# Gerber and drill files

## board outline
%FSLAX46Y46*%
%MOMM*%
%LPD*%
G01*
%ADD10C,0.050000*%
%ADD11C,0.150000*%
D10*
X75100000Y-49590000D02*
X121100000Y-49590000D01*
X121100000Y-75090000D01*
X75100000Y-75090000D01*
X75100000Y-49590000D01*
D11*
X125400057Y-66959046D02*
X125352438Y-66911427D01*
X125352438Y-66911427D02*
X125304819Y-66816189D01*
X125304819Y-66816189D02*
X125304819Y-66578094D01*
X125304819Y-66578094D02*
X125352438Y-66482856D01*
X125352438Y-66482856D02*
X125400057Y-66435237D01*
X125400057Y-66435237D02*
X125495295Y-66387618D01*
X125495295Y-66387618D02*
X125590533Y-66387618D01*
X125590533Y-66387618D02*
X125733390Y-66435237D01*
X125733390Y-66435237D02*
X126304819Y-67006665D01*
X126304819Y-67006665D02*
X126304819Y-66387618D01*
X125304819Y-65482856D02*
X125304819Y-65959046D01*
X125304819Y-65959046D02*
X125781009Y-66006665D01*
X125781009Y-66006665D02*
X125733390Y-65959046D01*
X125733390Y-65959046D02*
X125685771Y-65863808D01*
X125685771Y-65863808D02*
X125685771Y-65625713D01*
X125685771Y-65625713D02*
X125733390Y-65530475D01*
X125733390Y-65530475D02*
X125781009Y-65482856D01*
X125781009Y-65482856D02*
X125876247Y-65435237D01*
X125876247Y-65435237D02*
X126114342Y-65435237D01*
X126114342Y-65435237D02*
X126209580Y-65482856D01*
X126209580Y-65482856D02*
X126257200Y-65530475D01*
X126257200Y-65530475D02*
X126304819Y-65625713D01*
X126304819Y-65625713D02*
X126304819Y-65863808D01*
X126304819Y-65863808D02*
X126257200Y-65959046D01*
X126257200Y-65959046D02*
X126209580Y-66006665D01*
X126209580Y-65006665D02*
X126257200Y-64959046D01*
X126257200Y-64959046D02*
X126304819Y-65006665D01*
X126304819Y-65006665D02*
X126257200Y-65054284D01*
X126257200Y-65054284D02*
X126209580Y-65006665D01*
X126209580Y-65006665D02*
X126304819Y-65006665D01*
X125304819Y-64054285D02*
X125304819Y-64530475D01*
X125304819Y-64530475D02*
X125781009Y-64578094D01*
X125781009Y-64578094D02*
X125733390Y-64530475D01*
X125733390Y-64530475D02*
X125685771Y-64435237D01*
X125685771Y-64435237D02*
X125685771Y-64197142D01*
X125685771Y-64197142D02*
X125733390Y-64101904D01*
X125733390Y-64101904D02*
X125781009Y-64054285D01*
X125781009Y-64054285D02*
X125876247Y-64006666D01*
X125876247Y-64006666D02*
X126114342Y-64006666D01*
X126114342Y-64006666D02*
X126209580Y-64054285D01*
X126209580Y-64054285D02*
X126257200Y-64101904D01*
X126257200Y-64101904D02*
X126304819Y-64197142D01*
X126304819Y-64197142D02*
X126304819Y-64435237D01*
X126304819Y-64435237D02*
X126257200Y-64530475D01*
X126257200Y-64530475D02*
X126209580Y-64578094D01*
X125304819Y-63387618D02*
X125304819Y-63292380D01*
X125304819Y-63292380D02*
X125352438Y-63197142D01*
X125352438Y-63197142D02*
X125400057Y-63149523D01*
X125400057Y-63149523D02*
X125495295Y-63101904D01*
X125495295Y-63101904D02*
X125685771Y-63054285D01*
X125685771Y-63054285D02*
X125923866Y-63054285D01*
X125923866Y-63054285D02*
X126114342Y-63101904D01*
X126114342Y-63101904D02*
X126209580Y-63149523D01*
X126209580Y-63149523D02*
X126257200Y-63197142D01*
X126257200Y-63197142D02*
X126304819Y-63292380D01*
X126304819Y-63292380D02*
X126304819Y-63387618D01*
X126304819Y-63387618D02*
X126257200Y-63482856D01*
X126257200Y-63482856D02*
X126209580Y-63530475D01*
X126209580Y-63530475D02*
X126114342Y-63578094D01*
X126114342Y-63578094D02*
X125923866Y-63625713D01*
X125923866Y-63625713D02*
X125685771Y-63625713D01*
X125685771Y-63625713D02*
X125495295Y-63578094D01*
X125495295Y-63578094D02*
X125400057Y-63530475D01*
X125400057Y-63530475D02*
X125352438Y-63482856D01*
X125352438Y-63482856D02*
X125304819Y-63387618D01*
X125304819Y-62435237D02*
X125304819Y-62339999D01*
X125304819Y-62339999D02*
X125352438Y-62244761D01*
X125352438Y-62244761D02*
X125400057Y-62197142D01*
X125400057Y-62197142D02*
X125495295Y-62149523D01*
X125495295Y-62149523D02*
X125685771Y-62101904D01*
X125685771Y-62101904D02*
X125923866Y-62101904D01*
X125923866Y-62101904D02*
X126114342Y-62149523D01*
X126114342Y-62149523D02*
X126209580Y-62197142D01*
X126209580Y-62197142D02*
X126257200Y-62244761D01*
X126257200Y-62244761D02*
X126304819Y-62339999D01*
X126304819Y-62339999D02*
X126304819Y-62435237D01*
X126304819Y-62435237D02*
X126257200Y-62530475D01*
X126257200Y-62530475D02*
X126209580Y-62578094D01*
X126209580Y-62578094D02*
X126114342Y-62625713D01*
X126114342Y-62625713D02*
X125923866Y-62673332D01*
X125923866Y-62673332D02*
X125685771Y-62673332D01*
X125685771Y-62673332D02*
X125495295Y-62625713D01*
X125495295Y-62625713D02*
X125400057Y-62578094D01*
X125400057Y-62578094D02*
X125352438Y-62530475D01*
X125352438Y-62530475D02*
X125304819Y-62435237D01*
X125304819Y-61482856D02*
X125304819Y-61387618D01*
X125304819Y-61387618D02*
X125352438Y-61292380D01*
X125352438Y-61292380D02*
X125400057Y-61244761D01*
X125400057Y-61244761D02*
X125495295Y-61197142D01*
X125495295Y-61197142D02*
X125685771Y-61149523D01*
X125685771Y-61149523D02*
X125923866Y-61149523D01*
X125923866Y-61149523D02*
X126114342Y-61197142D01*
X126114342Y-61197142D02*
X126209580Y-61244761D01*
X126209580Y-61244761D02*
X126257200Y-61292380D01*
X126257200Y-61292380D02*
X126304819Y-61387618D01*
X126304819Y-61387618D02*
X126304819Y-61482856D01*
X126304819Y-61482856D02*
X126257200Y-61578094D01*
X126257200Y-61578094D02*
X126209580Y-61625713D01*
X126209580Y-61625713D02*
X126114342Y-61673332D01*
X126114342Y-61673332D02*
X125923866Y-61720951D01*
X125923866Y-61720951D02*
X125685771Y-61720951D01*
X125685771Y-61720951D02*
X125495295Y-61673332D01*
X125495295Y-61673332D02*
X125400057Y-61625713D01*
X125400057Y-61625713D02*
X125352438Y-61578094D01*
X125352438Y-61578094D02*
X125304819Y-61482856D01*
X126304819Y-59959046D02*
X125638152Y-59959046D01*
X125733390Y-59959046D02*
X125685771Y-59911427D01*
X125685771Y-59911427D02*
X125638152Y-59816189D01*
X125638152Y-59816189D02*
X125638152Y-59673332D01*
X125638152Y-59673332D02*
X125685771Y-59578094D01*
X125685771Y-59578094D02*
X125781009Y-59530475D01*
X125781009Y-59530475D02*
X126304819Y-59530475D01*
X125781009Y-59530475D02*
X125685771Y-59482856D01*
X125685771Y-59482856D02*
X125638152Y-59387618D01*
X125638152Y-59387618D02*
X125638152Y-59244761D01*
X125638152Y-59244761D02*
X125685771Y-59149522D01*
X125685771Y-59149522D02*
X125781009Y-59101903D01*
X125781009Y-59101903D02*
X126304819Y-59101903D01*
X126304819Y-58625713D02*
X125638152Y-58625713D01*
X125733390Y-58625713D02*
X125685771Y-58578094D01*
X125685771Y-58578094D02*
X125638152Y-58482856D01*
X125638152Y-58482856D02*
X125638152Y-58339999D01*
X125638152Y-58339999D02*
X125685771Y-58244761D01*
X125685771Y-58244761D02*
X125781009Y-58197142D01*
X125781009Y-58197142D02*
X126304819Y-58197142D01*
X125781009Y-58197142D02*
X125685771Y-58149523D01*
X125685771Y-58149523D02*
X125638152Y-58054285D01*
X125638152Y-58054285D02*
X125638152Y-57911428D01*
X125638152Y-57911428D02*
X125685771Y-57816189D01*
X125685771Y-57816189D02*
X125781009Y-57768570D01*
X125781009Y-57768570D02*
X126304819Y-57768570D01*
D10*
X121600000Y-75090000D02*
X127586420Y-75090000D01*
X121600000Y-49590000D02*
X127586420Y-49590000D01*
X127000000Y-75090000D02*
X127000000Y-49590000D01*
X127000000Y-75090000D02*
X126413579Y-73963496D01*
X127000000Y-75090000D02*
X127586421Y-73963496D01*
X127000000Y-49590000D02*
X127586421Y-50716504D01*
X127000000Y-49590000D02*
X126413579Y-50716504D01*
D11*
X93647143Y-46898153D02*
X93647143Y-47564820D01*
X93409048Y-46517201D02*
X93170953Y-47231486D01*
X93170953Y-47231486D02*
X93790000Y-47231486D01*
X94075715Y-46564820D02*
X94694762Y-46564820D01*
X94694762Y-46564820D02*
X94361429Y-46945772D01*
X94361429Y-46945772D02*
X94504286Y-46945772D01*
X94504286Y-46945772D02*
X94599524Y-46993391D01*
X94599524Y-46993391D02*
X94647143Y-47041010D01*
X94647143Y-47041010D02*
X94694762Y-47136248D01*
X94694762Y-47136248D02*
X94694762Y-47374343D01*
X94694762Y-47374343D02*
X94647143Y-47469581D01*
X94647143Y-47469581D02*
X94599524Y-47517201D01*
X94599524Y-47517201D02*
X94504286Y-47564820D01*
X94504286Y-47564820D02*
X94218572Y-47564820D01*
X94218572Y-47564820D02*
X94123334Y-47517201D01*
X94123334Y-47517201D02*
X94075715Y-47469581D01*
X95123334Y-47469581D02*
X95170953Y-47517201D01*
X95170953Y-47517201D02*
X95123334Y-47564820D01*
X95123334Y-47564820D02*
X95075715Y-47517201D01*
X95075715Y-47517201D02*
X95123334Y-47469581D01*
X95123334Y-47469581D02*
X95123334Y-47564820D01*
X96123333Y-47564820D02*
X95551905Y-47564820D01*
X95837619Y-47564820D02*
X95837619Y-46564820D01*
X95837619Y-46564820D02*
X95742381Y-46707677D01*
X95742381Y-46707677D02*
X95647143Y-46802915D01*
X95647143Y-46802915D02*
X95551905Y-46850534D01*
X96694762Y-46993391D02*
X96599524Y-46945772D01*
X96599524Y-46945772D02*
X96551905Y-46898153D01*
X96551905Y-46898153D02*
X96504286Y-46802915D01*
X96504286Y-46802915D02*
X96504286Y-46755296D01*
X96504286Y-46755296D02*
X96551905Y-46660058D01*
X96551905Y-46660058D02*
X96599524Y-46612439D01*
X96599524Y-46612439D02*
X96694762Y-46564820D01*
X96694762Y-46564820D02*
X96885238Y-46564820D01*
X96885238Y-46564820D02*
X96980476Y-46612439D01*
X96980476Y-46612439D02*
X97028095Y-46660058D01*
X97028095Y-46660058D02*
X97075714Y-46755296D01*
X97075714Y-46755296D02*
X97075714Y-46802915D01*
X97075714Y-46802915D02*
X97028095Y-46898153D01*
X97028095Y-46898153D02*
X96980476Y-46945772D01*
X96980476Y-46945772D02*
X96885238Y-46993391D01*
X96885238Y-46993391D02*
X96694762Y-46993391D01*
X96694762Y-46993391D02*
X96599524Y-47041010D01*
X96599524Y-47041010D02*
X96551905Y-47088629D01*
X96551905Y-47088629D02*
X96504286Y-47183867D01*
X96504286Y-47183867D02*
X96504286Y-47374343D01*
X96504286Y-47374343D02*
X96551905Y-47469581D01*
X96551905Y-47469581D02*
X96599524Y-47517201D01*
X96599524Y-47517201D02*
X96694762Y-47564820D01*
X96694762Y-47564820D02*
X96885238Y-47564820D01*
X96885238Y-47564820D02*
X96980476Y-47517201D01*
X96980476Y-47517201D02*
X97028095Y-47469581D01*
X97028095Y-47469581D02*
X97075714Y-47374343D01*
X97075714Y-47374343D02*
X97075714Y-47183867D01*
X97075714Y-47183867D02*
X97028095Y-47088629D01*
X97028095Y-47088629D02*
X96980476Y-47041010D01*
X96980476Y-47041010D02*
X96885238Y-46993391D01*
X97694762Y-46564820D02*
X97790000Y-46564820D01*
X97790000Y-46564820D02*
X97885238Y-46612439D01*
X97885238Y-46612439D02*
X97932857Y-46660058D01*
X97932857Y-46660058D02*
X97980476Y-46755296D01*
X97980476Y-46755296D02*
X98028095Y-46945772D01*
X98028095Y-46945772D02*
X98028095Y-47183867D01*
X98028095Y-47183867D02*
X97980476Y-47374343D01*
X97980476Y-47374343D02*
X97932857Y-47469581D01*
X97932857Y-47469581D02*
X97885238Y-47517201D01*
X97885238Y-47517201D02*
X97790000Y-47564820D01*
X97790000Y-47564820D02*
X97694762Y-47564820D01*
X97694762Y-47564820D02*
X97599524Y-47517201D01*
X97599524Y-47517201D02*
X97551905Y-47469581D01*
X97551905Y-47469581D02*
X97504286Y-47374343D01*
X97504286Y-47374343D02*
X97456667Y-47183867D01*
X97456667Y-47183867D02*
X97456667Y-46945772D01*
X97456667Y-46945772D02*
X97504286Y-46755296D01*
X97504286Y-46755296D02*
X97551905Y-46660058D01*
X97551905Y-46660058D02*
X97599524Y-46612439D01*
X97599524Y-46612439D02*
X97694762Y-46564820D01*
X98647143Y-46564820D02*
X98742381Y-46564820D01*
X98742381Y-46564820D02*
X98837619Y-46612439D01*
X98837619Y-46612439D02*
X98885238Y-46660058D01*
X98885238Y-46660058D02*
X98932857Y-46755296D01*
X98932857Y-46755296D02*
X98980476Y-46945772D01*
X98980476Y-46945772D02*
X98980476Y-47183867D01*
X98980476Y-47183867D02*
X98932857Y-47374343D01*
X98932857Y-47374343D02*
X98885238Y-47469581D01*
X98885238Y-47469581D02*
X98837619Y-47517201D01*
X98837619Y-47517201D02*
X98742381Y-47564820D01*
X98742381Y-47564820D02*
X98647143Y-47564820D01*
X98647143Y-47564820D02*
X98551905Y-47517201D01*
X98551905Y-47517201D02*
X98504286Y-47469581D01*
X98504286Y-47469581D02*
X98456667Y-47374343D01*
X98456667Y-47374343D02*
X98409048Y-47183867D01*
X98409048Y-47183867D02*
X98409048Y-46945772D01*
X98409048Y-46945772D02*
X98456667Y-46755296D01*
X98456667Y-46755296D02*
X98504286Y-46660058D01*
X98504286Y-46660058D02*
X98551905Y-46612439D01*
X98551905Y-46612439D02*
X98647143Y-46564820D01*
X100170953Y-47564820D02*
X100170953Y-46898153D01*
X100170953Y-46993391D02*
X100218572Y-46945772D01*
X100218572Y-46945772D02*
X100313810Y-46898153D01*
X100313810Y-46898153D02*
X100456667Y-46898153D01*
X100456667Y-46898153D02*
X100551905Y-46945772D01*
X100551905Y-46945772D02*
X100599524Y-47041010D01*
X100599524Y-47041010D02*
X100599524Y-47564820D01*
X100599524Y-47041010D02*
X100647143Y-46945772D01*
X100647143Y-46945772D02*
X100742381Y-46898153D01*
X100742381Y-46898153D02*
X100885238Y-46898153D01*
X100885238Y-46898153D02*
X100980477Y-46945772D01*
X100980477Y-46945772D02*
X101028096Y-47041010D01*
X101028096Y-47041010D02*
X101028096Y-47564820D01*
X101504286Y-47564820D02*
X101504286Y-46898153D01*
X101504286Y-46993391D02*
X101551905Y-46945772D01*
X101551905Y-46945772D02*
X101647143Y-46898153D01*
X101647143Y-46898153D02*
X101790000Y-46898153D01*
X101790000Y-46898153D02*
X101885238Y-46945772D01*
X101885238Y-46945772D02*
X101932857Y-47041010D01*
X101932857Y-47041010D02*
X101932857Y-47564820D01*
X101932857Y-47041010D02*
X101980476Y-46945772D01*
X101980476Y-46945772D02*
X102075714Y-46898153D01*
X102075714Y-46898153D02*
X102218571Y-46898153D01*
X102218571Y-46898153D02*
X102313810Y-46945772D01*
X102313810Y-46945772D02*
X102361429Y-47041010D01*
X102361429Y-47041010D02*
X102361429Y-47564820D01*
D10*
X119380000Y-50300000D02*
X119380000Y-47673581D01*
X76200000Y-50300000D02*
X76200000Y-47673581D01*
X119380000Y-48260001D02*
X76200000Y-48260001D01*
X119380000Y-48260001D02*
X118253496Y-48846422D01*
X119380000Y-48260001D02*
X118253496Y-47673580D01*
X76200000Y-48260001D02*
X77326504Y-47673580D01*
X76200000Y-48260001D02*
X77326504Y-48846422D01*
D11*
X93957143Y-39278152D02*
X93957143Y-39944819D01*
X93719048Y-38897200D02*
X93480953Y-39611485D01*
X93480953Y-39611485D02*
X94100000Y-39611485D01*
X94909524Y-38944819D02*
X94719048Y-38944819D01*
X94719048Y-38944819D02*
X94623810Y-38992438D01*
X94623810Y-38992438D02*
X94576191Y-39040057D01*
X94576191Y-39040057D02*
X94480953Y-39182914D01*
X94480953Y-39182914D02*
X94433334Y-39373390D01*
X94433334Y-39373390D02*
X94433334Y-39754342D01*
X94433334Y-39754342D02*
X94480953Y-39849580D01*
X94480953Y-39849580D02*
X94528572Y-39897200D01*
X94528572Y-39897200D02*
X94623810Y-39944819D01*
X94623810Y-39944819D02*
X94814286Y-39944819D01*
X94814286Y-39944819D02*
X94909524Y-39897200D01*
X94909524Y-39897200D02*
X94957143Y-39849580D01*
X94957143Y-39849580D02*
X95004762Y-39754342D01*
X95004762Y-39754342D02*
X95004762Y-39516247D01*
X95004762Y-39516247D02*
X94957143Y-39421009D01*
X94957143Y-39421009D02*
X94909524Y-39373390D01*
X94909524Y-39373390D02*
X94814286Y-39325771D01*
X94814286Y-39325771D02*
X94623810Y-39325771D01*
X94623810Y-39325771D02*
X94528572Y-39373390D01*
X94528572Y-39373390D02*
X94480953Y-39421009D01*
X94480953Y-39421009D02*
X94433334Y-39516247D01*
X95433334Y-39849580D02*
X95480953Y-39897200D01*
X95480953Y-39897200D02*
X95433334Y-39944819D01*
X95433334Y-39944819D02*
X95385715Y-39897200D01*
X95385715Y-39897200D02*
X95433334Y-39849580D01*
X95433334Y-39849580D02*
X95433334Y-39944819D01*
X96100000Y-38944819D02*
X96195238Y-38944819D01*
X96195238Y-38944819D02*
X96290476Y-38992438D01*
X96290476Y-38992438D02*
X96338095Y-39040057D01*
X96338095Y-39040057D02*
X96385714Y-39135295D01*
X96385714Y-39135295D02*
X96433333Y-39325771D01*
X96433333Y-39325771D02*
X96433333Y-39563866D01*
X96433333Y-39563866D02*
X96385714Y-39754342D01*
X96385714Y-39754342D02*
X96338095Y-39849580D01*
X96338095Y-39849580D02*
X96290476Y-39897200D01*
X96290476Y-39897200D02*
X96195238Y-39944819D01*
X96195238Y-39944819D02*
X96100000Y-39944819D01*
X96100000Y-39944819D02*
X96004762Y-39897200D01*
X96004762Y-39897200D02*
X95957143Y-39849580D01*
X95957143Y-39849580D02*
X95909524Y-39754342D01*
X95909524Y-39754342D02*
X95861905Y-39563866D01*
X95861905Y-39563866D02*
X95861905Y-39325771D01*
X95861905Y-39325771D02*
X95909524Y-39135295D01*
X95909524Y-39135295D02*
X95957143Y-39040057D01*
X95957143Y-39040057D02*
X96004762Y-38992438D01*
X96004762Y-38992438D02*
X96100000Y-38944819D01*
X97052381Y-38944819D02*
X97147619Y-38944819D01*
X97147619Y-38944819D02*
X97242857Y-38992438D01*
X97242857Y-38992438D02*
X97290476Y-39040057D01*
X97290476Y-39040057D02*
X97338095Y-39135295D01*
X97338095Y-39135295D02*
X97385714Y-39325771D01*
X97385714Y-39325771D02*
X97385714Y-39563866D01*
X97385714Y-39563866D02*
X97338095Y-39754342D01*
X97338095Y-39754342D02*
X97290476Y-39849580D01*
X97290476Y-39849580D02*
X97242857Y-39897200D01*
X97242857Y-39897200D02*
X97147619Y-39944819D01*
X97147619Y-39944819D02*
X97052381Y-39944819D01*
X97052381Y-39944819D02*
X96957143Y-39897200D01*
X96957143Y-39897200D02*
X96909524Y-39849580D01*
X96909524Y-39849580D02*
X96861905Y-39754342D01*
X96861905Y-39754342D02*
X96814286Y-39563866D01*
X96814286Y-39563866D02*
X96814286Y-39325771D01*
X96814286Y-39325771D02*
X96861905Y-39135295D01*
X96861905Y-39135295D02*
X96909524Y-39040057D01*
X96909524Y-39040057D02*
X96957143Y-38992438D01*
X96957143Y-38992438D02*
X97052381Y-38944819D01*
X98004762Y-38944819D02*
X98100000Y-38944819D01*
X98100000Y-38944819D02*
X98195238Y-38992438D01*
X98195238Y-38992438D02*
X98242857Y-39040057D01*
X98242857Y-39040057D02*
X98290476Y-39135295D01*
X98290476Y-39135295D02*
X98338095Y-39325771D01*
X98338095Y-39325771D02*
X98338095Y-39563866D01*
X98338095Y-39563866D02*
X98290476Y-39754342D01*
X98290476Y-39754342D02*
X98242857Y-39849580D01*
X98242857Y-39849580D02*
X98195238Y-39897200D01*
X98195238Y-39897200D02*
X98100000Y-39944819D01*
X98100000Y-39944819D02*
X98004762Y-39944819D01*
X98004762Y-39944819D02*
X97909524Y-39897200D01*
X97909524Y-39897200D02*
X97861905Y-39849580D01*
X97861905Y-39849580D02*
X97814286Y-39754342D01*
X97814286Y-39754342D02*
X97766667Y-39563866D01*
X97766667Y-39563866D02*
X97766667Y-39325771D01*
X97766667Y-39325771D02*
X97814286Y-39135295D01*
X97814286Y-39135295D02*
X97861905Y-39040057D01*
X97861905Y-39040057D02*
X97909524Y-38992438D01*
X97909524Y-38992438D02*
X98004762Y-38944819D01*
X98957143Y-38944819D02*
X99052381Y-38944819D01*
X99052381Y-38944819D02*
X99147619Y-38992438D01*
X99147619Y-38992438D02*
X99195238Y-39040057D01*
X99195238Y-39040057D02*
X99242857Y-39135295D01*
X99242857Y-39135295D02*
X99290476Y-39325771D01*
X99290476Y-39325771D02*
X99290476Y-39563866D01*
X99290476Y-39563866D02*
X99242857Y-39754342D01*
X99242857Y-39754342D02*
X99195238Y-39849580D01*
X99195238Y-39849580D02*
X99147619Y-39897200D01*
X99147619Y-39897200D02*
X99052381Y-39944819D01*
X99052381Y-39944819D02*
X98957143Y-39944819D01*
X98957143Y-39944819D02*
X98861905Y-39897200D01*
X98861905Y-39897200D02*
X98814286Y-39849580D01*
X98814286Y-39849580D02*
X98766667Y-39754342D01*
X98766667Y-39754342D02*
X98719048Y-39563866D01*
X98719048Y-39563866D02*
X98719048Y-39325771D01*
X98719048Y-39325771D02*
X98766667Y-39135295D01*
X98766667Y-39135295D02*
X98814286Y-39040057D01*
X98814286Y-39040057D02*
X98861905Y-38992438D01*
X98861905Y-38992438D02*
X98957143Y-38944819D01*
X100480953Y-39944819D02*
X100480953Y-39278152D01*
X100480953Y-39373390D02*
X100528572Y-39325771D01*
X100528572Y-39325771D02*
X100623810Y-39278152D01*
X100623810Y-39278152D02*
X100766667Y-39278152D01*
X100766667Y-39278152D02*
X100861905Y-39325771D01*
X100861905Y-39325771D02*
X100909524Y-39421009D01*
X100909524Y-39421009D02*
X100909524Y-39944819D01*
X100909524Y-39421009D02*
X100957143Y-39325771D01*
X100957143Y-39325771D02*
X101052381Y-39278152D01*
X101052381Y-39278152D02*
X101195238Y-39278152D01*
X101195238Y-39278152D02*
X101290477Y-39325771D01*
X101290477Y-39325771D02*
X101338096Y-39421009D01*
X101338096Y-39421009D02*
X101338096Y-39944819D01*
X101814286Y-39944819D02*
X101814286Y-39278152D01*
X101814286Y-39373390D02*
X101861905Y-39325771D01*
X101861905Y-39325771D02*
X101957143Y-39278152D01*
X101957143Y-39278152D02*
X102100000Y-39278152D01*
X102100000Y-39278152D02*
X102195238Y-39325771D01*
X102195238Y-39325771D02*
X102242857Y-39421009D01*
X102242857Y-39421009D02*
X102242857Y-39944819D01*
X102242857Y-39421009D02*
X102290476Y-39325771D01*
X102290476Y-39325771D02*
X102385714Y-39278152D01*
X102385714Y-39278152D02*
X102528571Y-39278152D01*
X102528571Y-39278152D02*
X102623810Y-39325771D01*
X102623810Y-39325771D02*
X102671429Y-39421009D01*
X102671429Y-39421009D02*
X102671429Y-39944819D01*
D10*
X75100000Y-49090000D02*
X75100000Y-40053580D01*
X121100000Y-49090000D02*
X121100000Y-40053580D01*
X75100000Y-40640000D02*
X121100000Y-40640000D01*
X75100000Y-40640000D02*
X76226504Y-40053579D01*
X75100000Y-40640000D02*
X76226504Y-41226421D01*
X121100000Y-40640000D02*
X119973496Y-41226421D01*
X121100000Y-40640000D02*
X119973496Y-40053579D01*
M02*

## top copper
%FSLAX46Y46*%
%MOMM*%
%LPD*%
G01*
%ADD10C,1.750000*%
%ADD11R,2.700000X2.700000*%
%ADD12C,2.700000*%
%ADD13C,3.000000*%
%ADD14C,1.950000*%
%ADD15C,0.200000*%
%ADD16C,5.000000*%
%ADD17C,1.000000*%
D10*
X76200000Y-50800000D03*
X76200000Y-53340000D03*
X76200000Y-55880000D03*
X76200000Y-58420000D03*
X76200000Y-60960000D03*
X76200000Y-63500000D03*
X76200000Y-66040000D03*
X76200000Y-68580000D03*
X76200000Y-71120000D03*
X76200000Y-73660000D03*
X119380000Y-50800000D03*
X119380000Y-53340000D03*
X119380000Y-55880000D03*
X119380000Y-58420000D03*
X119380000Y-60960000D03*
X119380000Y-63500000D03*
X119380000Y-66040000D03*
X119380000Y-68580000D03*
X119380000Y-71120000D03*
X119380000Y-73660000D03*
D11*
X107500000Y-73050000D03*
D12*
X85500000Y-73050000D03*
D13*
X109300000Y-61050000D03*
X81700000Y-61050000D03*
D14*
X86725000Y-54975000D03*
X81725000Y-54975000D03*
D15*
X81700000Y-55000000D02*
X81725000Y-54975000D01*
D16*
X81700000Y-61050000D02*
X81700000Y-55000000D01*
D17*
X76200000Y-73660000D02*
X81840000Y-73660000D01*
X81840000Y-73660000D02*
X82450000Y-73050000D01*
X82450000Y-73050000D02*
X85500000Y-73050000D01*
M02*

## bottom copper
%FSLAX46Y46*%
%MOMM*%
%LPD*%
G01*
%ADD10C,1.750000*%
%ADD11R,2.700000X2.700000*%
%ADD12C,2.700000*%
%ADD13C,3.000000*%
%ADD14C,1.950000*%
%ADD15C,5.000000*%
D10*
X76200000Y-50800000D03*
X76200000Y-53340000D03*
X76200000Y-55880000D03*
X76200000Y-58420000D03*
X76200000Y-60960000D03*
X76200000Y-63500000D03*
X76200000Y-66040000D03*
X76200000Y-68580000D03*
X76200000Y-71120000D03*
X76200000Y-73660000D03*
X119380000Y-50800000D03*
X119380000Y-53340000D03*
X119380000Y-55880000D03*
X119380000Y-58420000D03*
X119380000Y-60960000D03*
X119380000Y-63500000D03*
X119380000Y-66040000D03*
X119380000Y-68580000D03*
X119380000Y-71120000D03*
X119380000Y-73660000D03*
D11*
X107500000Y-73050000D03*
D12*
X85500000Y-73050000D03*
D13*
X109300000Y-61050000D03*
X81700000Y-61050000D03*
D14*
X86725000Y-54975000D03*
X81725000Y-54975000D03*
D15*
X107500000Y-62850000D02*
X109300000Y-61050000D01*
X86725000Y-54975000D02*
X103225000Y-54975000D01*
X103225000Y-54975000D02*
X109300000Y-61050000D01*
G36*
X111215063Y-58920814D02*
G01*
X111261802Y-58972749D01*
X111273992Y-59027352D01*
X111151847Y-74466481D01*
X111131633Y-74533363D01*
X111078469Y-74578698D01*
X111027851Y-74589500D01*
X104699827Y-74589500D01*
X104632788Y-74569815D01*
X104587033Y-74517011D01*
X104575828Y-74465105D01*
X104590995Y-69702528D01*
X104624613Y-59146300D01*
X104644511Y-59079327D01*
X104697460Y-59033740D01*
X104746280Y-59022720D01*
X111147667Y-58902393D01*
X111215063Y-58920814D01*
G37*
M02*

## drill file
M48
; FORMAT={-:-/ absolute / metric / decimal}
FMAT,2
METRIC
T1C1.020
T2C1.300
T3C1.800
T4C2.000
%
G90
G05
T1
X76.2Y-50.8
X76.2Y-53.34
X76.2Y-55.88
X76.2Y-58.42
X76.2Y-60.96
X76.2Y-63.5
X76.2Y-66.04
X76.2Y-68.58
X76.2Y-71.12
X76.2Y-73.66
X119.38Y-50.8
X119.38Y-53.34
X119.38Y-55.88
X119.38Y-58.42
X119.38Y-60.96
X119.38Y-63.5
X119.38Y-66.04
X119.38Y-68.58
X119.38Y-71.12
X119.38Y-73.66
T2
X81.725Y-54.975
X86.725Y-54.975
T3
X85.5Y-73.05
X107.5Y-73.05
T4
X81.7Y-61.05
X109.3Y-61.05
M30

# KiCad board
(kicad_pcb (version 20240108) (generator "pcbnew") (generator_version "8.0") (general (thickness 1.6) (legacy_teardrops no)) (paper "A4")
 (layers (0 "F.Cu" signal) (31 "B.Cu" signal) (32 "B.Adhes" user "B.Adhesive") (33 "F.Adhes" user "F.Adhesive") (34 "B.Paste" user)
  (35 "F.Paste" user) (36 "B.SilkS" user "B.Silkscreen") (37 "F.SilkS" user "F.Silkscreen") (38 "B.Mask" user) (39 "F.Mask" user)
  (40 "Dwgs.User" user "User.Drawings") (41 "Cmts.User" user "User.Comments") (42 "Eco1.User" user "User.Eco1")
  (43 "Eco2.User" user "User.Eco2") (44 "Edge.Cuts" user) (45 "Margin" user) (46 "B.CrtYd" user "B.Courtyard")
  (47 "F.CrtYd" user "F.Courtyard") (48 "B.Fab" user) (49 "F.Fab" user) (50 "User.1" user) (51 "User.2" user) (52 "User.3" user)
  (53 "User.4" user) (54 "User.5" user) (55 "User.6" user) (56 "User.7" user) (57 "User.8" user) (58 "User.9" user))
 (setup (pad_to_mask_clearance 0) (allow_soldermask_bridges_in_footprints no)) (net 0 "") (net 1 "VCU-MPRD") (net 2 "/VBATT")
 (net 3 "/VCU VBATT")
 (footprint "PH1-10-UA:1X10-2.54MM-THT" (layer "F.Cu") (at 76.2 50.8 -90)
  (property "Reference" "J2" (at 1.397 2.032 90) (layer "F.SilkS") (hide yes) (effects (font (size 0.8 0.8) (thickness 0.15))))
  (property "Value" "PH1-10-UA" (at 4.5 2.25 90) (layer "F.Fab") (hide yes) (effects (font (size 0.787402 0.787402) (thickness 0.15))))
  (pad "1" thru_hole circle (at 0 0 270) (size 1.75 1.75) (drill 1.02) (layers "*.Cu" "*.Mask") (remove_unused_layers no)
   (solder_mask_margin 0.102))
  (pad "2" thru_hole circle (at 2.54 0 270) (size 1.75 1.75) (drill 1.02) (layers "*.Cu" "*.Mask") (remove_unused_layers no)
   (solder_mask_margin 0.102))
  (pad "3" thru_hole circle (at 5.08 0 270) (size 1.75 1.75) (drill 1.02) (layers "*.Cu" "*.Mask") (remove_unused_layers no)
   (solder_mask_margin 0.102))
  (pad "4" thru_hole circle (at 7.62 0 270) (size 1.75 1.75) (drill 1.02) (layers "*.Cu" "*.Mask") (remove_unused_layers no)
   (solder_mask_margin 0.102))
  (pad "5" thru_hole circle (at 10.16 0 270) (size 1.75 1.75) (drill 1.02) (layers "*.Cu" "*.Mask") (remove_unused_layers no)
   (solder_mask_margin 0.102))
  (pad "6" thru_hole circle (at 12.7 0 270) (size 1.75 1.75) (drill 1.02) (layers "*.Cu" "*.Mask") (remove_unused_layers no)
   (solder_mask_margin 0.102))
  (pad "7" thru_hole circle (at 15.24 0 270) (size 1.75 1.75) (drill 1.02) (layers "*.Cu" "*.Mask") (remove_unused_layers no)
   (solder_mask_margin 0.102))
  (pad "8" thru_hole circle (at 17.78 0 270) (size 1.75 1.75) (drill 1.02) (layers "*.Cu" "*.Mask") (remove_unused_layers no)
   (solder_mask_margin 0.102))
  (pad "9" thru_hole circle (at 20.32 0 270) (size 1.75 1.75) (drill 1.02) (layers "*.Cu" "*.Mask") (remove_unused_layers no)
   (solder_mask_margin 0.102))
  (pad "10" thru_hole circle (at 22.86 0 270) (size 1.75 1.75) (drill 1.02) (layers "*.Cu" "*.Mask") (remove_unused_layers no)
   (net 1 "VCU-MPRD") (solder_mask_margin 0.102)))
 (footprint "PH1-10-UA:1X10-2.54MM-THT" (layer "F.Cu") (at 119.38 50.8 -90)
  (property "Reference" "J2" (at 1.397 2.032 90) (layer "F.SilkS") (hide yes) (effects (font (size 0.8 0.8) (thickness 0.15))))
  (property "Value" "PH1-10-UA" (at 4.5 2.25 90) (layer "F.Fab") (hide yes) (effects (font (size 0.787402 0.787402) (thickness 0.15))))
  (pad "1" thru_hole circle (at 0 0 270) (size 1.75 1.75) (drill 1.02) (layers "*.Cu" "*.Mask") (remove_unused_layers no)
   (solder_mask_margin 0.102))
  (pad "2" thru_hole circle (at 2.54 0 270) (size 1.75 1.75) (drill 1.02) (layers "*.Cu" "*.Mask") (remove_unused_layers no)
   (solder_mask_margin 0.102))
  (pad "3" thru_hole circle (at 5.08 0 270) (size 1.75 1.75) (drill 1.02) (layers "*.Cu" "*.Mask") (remove_unused_layers no)
   (solder_mask_margin 0.102))
  (pad "4" thru_hole circle (at 7.62 0 270) (size 1.75 1.75) (drill 1.02) (layers "*.Cu" "*.Mask") (remove_unused_layers no)
   (solder_mask_margin 0.102))
  (pad "5" thru_hole circle (at 10.16 0 270) (size 1.75 1.75) (drill 1.02) (layers "*.Cu" "*.Mask") (remove_unused_layers no)
   (solder_mask_margin 0.102))
  (pad "6" thru_hole circle (at 12.7 0 270) (size 1.75 1.75) (drill 1.02) (layers "*.Cu" "*.Mask") (remove_unused_layers no)
   (solder_mask_margin 0.102))
  (pad "7" thru_hole circle (at 15.24 0 270) (size 1.75 1.75) (drill 1.02) (layers "*.Cu" "*.Mask") (remove_unused_layers no)
   (solder_mask_margin 0.102))
  (pad "8" thru_hole circle (at 17.78 0 270) (size 1.75 1.75) (drill 1.02) (layers "*.Cu" "*.Mask") (remove_unused_layers no)
   (solder_mask_margin 0.102))
  (pad "9" thru_hole circle (at 20.32 0 270) (size 1.75 1.75) (drill 1.02) (layers "*.Cu" "*.Mask") (remove_unused_layers no)
   (solder_mask_margin 0.102))
  (pad "10" thru_hole circle (at 22.86 0 270) (size 1.75 1.75) (drill 1.02) (layers "*.Cu" "*.Mask") (remove_unused_layers no)
   (solder_mask_margin 0.102)))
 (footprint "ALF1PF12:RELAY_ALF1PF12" (layer "F.Cu") (at 95.5 67.05 180)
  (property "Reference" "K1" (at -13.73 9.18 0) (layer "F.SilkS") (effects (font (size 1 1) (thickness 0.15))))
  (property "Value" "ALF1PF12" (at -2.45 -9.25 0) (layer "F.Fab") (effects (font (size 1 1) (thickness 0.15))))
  (pad "1" thru_hole rect (at -12 -6 180) (size 2.7 2.7) (drill 1.8) (layers "*.Cu" "*.Mask") (remove_unused_layers no) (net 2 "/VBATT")
   (solder_mask_margin 0.102))
  (pad "2" thru_hole circle (at 10 -6 180) (size 2.7 2.7) (drill 1.8) (layers "*.Cu" "*.Mask") (remove_unused_layers no) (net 1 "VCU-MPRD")
   (solder_mask_margin 0.102))
  (pad "3" thru_hole circle (at -13.8 6 180) (size 3 3) (drill 2) (layers "*.Cu" "*.Mask") (remove_unused_layers no) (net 2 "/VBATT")
   (solder_mask_margin 0.102))
  (pad "4" thru_hole circle (at 13.8 6 180) (size 3 3) (drill 2) (layers "*.Cu" "*.Mask") (remove_unused_layers no) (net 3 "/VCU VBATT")
   (solder_mask_margin 0.102)))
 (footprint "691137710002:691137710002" (layer "F.Cu") (at 84.225 54.975 180)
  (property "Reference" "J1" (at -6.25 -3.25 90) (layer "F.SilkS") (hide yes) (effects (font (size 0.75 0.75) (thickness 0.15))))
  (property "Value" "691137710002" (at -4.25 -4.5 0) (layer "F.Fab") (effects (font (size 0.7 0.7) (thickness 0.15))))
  (pad "1" thru_hole circle (at -2.5 0 180) (size 1.95 1.95) (drill 1.3) (layers "*.Cu" "*.Mask") (remove_unused_layers no) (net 2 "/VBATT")
   (solder_mask_margin 0.102))
  (pad "2" thru_hole circle (at 2.5 0 180) (size 1.95 1.95) (drill 1.3) (layers "*.Cu" "*.Mask") (remove_unused_layers no)
   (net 3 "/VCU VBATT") (solder_mask_margin 0.102)))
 (gr_rect (start 75.1 49.59) (end 121.1 75.09) (stroke (width 0.05) (type default)) (fill none) (layer "Edge.Cuts"))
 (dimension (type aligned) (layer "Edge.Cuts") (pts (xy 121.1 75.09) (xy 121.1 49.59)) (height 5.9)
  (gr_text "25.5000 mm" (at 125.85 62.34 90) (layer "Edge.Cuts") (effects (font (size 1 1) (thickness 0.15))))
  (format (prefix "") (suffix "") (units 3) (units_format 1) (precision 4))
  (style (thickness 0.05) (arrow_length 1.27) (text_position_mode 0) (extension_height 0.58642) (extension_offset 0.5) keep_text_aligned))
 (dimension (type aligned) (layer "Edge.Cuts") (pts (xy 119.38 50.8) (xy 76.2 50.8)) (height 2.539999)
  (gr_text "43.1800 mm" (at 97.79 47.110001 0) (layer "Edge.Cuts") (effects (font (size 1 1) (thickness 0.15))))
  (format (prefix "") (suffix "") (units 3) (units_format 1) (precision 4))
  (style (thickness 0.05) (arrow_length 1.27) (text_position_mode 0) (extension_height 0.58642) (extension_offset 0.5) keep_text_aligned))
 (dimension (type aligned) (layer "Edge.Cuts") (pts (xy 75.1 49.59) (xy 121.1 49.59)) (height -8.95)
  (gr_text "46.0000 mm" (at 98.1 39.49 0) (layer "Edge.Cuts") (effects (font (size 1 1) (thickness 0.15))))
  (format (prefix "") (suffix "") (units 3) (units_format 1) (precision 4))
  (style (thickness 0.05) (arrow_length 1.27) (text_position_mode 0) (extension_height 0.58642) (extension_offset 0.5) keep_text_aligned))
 (segment (start 107.5 62.85) (end 109.3 61.05) (width 5) (layer "B.Cu") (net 2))
 (segment (start 86.725 54.975) (end 103.225 54.975) (width 5) (layer "B.Cu") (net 2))
 (segment (start 103.225 54.975) (end 109.3 61.05) (width 5) (layer "B.Cu") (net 2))
 (segment (start 81.7 55) (end 81.725 54.975) (width 0.2) (layer "F.Cu") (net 3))
 (segment (start 81.7 61.05) (end 81.7 55) (width 5) (layer "F.Cu") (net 3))
 (segment (start 76.2 73.66) (end 81.84 73.66) (width 1) (layer "F.Cu") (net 1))
 (segment (start 81.84 73.66) (end 82.45 73.05) (width 1) (layer "F.Cu") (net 1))
 (segment (start 82.45 73.05) (end 85.5 73.05) (width 1) (layer "F.Cu") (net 1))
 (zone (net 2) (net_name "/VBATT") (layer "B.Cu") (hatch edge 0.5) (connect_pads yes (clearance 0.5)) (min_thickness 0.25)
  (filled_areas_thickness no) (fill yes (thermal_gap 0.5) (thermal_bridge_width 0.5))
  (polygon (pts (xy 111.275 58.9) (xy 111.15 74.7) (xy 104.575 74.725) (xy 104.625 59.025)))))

